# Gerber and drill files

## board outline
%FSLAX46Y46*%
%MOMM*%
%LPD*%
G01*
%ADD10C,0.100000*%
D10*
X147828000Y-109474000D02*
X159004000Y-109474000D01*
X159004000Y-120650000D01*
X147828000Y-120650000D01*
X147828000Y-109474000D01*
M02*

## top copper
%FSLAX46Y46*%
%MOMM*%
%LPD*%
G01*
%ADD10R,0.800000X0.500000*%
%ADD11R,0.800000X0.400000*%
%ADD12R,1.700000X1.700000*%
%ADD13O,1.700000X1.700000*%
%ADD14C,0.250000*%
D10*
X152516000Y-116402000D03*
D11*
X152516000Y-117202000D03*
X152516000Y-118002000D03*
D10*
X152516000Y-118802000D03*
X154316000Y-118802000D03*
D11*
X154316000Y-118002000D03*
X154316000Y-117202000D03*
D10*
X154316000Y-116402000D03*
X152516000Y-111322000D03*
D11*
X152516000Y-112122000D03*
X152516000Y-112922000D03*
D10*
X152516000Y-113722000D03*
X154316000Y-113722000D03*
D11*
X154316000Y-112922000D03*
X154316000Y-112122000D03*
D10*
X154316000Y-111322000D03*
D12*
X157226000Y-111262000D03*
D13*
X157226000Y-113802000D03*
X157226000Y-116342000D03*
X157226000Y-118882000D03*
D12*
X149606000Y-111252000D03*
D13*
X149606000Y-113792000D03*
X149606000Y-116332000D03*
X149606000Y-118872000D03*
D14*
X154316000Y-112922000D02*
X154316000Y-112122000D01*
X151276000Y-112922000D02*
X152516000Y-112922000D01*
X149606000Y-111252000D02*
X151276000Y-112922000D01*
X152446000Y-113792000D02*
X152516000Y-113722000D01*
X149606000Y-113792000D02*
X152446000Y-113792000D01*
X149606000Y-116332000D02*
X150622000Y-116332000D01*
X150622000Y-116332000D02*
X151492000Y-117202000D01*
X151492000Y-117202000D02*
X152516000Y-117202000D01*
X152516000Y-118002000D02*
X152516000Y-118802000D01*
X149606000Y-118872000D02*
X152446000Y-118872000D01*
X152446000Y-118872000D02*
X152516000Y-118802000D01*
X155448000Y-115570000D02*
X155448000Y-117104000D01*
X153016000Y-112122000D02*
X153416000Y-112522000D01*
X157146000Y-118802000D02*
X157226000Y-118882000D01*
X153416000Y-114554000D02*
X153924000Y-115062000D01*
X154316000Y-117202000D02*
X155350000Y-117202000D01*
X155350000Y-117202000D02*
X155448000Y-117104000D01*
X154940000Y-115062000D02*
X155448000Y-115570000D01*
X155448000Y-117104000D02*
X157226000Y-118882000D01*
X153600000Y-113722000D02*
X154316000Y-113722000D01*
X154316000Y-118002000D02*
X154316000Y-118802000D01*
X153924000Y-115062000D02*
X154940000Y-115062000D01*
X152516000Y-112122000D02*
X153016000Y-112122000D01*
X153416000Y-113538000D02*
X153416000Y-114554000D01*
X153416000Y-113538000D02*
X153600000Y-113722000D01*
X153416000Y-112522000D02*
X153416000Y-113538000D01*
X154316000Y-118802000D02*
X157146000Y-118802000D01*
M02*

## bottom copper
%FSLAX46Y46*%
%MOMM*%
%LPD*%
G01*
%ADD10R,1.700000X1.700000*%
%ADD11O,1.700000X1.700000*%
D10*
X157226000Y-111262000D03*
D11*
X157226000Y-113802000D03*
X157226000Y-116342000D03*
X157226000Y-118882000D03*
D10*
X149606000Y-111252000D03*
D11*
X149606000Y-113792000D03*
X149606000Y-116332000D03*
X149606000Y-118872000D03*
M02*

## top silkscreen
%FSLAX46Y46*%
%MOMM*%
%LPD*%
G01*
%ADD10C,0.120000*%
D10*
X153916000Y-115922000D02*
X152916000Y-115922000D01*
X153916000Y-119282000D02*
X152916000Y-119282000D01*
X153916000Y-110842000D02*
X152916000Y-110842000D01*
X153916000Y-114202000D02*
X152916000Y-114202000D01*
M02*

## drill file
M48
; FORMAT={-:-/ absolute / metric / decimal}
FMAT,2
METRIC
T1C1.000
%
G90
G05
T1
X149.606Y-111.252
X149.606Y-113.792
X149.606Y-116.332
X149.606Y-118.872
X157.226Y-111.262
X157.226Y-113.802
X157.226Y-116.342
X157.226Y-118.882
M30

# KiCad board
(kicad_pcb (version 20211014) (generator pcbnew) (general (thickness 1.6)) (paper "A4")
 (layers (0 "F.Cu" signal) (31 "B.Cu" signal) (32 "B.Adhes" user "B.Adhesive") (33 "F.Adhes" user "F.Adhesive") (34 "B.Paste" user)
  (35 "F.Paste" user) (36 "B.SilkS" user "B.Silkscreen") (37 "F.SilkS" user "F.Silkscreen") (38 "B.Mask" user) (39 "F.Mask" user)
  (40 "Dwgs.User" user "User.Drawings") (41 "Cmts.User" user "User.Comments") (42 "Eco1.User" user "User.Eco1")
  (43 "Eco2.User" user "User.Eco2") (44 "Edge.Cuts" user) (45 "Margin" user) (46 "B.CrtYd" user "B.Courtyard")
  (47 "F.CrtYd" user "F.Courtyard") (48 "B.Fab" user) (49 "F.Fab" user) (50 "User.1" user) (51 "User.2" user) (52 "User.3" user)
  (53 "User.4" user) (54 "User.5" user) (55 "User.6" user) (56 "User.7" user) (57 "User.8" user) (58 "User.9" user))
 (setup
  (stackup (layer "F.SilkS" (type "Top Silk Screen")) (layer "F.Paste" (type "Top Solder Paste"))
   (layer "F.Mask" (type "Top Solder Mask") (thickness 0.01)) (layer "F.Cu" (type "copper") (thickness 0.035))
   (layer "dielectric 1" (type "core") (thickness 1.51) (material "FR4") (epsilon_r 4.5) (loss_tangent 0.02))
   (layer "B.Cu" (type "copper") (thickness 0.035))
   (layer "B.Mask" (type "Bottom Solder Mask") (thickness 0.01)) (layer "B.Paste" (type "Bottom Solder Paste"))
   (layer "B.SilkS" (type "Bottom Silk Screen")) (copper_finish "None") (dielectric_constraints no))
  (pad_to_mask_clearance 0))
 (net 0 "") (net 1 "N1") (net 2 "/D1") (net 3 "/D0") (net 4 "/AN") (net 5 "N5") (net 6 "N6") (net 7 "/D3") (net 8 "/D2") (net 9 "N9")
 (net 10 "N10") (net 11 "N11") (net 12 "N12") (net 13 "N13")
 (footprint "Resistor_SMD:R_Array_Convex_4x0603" (layer "F.Cu") (at 153.416 117.602)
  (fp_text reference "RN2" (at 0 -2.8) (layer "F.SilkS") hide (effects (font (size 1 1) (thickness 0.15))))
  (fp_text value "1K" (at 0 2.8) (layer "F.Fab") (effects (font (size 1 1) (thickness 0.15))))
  (fp_line (start 0.5 -1.68) (end -0.5 -1.68) (layer "F.SilkS") (width 0.12))
  (fp_line (start 0.5 1.68) (end -0.5 1.68) (layer "F.SilkS") (width 0.12))
  (pad "1" smd rect (at -0.9 -1.2) (size 0.8 0.5) (layers "F.Cu" "F.Paste" "F.Mask") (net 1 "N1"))
  (pad "2" smd rect (at -0.9 -0.4) (size 0.8 0.4) (layers "F.Cu" "F.Paste" "F.Mask") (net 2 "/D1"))
  (pad "3" smd rect (at -0.9 0.4) (size 0.8 0.4) (layers "F.Cu" "F.Paste" "F.Mask") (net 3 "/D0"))
  (pad "4" smd rect (at -0.9 1.2) (size 0.8 0.5) (layers "F.Cu" "F.Paste" "F.Mask") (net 3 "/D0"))
  (pad "5" smd rect (at 0.9 1.2) (size 0.8 0.5) (layers "F.Cu" "F.Paste" "F.Mask") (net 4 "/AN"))
  (pad "6" smd rect (at 0.9 0.4) (size 0.8 0.4) (layers "F.Cu" "F.Paste" "F.Mask") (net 4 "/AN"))
  (pad "7" smd rect (at 0.9 -0.4) (size 0.8 0.4) (layers "F.Cu" "F.Paste" "F.Mask") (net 4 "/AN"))
  (pad "8" smd rect (at 0.9 -1.2) (size 0.8 0.5) (layers "F.Cu" "F.Paste" "F.Mask") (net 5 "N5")))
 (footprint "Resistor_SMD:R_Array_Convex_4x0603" (layer "F.Cu") (at 153.416 112.522)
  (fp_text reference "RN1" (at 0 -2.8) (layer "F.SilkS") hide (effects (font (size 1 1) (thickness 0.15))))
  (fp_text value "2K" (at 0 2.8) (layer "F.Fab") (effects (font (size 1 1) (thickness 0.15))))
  (fp_line (start 0.5 -1.68) (end -0.5 -1.68) (layer "F.SilkS") (width 0.12))
  (fp_line (start 0.5 1.68) (end -0.5 1.68) (layer "F.SilkS") (width 0.12))
  (pad "1" smd rect (at -0.9 -1.2) (size 0.8 0.5) (layers "F.Cu" "F.Paste" "F.Mask") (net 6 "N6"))
  (pad "2" smd rect (at -0.9 -0.4) (size 0.8 0.4) (layers "F.Cu" "F.Paste" "F.Mask") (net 4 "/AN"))
  (pad "3" smd rect (at -0.9 0.4) (size 0.8 0.4) (layers "F.Cu" "F.Paste" "F.Mask") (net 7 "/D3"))
  (pad "4" smd rect (at -0.9 1.2) (size 0.8 0.5) (layers "F.Cu" "F.Paste" "F.Mask") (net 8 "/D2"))
  (pad "5" smd rect (at 0.9 1.2) (size 0.8 0.5) (layers "F.Cu" "F.Paste" "F.Mask") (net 4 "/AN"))
  (pad "6" smd rect (at 0.9 0.4) (size 0.8 0.4) (layers "F.Cu" "F.Paste" "F.Mask") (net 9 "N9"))
  (pad "7" smd rect (at 0.9 -0.4) (size 0.8 0.4) (layers "F.Cu" "F.Paste" "F.Mask") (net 9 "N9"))
  (pad "8" smd rect (at 0.9 -1.2) (size 0.8 0.5) (layers "F.Cu" "F.Paste" "F.Mask") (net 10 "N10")))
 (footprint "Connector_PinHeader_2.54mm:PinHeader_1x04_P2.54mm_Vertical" (layer "B.Cu") (at 157.226 111.262 180)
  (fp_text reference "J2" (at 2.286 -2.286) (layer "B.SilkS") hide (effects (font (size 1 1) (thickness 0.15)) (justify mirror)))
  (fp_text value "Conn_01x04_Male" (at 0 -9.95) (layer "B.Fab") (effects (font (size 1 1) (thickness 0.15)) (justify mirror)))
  (pad "1" thru_hole rect (at 0 0 180) (size 1.7 1.7) (drill 1) (layers *.Cu *.Mask) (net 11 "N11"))
  (pad "2" thru_hole oval (at 0 -2.54 180) (size 1.7 1.7) (drill 1) (layers *.Cu *.Mask) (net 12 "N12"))
  (pad "3" thru_hole oval (at 0 -5.08 180) (size 1.7 1.7) (drill 1) (layers *.Cu *.Mask) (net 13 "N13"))
  (pad "4" thru_hole oval (at 0 -7.62 180) (size 1.7 1.7) (drill 1) (layers *.Cu *.Mask) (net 4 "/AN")))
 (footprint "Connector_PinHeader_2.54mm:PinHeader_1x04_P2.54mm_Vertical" (layer "B.Cu") (at 149.606 111.252 180)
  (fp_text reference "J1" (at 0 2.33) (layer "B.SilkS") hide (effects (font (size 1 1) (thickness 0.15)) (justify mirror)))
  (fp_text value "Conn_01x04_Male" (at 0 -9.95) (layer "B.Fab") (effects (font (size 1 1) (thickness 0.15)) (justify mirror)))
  (pad "1" thru_hole rect (at 0 0 180) (size 1.7 1.7) (drill 1) (layers *.Cu *.Mask) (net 7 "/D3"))
  (pad "2" thru_hole oval (at 0 -2.54 180) (size 1.7 1.7) (drill 1) (layers *.Cu *.Mask) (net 8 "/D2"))
  (pad "3" thru_hole oval (at 0 -5.08 180) (size 1.7 1.7) (drill 1) (layers *.Cu *.Mask) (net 2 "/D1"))
  (pad "4" thru_hole oval (at 0 -7.62 180) (size 1.7 1.7) (drill 1) (layers *.Cu *.Mask) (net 3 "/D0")))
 (gr_rect (start 147.828 120.65) (end 159.004 109.474) (layer "Edge.Cuts") (width 0.1) (fill none))
 (segment (start 154.316 112.922) (end 154.316 112.122) (width 0.25) (layer "F.Cu") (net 9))
 (segment (start 151.276 112.922) (end 152.516 112.922) (width 0.25) (layer "F.Cu") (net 7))
 (segment (start 149.606 111.252) (end 151.276 112.922) (width 0.25) (layer "F.Cu") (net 7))
 (segment (start 152.446 113.792) (end 152.516 113.722) (width 0.25) (layer "F.Cu") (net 8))
 (segment (start 149.606 113.792) (end 152.446 113.792) (width 0.25) (layer "F.Cu") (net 8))
 (segment (start 149.606 116.332) (end 150.622 116.332) (width 0.25) (layer "F.Cu") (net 2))
 (segment (start 150.622 116.332) (end 151.492 117.202) (width 0.25) (layer "F.Cu") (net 2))
 (segment (start 151.492 117.202) (end 152.516 117.202) (width 0.25) (layer "F.Cu") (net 2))
 (segment (start 152.516 118.002) (end 152.516 118.802) (width 0.25) (layer "F.Cu") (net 3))
 (segment (start 149.606 118.872) (end 152.446 118.872) (width 0.25) (layer "F.Cu") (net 3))
 (segment (start 152.446 118.872) (end 152.516 118.802) (width 0.25) (layer "F.Cu") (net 3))
 (segment (start 155.448 115.57) (end 155.448 117.104) (width 0.25) (layer "F.Cu") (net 4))
 (segment (start 153.016 112.122) (end 153.416 112.522) (width 0.25) (layer "F.Cu") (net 4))
 (segment (start 157.146 118.802) (end 157.226 118.882) (width 0.25) (layer "F.Cu") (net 4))
 (segment (start 153.416 114.554) (end 153.924 115.062) (width 0.25) (layer "F.Cu") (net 4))
 (segment (start 154.316 117.202) (end 155.35 117.202) (width 0.25) (layer "F.Cu") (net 4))
 (segment (start 155.35 117.202) (end 155.448 117.104) (width 0.25) (layer "F.Cu") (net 4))
 (segment (start 154.94 115.062) (end 155.448 115.57) (width 0.25) (layer "F.Cu") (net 4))
 (segment (start 155.448 117.104) (end 157.226 118.882) (width 0.25) (layer "F.Cu") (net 4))
 (segment (start 153.6 113.722) (end 154.316 113.722) (width 0.25) (layer "F.Cu") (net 4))
 (segment (start 154.316 118.002) (end 154.316 118.802) (width 0.25) (layer "F.Cu") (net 4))
 (segment (start 153.924 115.062) (end 154.94 115.062) (width 0.25) (layer "F.Cu") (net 4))
 (segment (start 152.516 112.122) (end 153.016 112.122) (width 0.25) (layer "F.Cu") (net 4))
 (segment (start 153.416 113.538) (end 153.416 114.554) (width 0.25) (layer "F.Cu") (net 4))
 (segment (start 153.416 113.538) (end 153.6 113.722) (width 0.25) (layer "F.Cu") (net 4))
 (segment (start 153.416 112.522) (end 153.416 113.538) (width 0.25) (layer "F.Cu") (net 4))
 (segment (start 154.316 118.802) (end 157.146 118.802) (width 0.25) (layer "F.Cu") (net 4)))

